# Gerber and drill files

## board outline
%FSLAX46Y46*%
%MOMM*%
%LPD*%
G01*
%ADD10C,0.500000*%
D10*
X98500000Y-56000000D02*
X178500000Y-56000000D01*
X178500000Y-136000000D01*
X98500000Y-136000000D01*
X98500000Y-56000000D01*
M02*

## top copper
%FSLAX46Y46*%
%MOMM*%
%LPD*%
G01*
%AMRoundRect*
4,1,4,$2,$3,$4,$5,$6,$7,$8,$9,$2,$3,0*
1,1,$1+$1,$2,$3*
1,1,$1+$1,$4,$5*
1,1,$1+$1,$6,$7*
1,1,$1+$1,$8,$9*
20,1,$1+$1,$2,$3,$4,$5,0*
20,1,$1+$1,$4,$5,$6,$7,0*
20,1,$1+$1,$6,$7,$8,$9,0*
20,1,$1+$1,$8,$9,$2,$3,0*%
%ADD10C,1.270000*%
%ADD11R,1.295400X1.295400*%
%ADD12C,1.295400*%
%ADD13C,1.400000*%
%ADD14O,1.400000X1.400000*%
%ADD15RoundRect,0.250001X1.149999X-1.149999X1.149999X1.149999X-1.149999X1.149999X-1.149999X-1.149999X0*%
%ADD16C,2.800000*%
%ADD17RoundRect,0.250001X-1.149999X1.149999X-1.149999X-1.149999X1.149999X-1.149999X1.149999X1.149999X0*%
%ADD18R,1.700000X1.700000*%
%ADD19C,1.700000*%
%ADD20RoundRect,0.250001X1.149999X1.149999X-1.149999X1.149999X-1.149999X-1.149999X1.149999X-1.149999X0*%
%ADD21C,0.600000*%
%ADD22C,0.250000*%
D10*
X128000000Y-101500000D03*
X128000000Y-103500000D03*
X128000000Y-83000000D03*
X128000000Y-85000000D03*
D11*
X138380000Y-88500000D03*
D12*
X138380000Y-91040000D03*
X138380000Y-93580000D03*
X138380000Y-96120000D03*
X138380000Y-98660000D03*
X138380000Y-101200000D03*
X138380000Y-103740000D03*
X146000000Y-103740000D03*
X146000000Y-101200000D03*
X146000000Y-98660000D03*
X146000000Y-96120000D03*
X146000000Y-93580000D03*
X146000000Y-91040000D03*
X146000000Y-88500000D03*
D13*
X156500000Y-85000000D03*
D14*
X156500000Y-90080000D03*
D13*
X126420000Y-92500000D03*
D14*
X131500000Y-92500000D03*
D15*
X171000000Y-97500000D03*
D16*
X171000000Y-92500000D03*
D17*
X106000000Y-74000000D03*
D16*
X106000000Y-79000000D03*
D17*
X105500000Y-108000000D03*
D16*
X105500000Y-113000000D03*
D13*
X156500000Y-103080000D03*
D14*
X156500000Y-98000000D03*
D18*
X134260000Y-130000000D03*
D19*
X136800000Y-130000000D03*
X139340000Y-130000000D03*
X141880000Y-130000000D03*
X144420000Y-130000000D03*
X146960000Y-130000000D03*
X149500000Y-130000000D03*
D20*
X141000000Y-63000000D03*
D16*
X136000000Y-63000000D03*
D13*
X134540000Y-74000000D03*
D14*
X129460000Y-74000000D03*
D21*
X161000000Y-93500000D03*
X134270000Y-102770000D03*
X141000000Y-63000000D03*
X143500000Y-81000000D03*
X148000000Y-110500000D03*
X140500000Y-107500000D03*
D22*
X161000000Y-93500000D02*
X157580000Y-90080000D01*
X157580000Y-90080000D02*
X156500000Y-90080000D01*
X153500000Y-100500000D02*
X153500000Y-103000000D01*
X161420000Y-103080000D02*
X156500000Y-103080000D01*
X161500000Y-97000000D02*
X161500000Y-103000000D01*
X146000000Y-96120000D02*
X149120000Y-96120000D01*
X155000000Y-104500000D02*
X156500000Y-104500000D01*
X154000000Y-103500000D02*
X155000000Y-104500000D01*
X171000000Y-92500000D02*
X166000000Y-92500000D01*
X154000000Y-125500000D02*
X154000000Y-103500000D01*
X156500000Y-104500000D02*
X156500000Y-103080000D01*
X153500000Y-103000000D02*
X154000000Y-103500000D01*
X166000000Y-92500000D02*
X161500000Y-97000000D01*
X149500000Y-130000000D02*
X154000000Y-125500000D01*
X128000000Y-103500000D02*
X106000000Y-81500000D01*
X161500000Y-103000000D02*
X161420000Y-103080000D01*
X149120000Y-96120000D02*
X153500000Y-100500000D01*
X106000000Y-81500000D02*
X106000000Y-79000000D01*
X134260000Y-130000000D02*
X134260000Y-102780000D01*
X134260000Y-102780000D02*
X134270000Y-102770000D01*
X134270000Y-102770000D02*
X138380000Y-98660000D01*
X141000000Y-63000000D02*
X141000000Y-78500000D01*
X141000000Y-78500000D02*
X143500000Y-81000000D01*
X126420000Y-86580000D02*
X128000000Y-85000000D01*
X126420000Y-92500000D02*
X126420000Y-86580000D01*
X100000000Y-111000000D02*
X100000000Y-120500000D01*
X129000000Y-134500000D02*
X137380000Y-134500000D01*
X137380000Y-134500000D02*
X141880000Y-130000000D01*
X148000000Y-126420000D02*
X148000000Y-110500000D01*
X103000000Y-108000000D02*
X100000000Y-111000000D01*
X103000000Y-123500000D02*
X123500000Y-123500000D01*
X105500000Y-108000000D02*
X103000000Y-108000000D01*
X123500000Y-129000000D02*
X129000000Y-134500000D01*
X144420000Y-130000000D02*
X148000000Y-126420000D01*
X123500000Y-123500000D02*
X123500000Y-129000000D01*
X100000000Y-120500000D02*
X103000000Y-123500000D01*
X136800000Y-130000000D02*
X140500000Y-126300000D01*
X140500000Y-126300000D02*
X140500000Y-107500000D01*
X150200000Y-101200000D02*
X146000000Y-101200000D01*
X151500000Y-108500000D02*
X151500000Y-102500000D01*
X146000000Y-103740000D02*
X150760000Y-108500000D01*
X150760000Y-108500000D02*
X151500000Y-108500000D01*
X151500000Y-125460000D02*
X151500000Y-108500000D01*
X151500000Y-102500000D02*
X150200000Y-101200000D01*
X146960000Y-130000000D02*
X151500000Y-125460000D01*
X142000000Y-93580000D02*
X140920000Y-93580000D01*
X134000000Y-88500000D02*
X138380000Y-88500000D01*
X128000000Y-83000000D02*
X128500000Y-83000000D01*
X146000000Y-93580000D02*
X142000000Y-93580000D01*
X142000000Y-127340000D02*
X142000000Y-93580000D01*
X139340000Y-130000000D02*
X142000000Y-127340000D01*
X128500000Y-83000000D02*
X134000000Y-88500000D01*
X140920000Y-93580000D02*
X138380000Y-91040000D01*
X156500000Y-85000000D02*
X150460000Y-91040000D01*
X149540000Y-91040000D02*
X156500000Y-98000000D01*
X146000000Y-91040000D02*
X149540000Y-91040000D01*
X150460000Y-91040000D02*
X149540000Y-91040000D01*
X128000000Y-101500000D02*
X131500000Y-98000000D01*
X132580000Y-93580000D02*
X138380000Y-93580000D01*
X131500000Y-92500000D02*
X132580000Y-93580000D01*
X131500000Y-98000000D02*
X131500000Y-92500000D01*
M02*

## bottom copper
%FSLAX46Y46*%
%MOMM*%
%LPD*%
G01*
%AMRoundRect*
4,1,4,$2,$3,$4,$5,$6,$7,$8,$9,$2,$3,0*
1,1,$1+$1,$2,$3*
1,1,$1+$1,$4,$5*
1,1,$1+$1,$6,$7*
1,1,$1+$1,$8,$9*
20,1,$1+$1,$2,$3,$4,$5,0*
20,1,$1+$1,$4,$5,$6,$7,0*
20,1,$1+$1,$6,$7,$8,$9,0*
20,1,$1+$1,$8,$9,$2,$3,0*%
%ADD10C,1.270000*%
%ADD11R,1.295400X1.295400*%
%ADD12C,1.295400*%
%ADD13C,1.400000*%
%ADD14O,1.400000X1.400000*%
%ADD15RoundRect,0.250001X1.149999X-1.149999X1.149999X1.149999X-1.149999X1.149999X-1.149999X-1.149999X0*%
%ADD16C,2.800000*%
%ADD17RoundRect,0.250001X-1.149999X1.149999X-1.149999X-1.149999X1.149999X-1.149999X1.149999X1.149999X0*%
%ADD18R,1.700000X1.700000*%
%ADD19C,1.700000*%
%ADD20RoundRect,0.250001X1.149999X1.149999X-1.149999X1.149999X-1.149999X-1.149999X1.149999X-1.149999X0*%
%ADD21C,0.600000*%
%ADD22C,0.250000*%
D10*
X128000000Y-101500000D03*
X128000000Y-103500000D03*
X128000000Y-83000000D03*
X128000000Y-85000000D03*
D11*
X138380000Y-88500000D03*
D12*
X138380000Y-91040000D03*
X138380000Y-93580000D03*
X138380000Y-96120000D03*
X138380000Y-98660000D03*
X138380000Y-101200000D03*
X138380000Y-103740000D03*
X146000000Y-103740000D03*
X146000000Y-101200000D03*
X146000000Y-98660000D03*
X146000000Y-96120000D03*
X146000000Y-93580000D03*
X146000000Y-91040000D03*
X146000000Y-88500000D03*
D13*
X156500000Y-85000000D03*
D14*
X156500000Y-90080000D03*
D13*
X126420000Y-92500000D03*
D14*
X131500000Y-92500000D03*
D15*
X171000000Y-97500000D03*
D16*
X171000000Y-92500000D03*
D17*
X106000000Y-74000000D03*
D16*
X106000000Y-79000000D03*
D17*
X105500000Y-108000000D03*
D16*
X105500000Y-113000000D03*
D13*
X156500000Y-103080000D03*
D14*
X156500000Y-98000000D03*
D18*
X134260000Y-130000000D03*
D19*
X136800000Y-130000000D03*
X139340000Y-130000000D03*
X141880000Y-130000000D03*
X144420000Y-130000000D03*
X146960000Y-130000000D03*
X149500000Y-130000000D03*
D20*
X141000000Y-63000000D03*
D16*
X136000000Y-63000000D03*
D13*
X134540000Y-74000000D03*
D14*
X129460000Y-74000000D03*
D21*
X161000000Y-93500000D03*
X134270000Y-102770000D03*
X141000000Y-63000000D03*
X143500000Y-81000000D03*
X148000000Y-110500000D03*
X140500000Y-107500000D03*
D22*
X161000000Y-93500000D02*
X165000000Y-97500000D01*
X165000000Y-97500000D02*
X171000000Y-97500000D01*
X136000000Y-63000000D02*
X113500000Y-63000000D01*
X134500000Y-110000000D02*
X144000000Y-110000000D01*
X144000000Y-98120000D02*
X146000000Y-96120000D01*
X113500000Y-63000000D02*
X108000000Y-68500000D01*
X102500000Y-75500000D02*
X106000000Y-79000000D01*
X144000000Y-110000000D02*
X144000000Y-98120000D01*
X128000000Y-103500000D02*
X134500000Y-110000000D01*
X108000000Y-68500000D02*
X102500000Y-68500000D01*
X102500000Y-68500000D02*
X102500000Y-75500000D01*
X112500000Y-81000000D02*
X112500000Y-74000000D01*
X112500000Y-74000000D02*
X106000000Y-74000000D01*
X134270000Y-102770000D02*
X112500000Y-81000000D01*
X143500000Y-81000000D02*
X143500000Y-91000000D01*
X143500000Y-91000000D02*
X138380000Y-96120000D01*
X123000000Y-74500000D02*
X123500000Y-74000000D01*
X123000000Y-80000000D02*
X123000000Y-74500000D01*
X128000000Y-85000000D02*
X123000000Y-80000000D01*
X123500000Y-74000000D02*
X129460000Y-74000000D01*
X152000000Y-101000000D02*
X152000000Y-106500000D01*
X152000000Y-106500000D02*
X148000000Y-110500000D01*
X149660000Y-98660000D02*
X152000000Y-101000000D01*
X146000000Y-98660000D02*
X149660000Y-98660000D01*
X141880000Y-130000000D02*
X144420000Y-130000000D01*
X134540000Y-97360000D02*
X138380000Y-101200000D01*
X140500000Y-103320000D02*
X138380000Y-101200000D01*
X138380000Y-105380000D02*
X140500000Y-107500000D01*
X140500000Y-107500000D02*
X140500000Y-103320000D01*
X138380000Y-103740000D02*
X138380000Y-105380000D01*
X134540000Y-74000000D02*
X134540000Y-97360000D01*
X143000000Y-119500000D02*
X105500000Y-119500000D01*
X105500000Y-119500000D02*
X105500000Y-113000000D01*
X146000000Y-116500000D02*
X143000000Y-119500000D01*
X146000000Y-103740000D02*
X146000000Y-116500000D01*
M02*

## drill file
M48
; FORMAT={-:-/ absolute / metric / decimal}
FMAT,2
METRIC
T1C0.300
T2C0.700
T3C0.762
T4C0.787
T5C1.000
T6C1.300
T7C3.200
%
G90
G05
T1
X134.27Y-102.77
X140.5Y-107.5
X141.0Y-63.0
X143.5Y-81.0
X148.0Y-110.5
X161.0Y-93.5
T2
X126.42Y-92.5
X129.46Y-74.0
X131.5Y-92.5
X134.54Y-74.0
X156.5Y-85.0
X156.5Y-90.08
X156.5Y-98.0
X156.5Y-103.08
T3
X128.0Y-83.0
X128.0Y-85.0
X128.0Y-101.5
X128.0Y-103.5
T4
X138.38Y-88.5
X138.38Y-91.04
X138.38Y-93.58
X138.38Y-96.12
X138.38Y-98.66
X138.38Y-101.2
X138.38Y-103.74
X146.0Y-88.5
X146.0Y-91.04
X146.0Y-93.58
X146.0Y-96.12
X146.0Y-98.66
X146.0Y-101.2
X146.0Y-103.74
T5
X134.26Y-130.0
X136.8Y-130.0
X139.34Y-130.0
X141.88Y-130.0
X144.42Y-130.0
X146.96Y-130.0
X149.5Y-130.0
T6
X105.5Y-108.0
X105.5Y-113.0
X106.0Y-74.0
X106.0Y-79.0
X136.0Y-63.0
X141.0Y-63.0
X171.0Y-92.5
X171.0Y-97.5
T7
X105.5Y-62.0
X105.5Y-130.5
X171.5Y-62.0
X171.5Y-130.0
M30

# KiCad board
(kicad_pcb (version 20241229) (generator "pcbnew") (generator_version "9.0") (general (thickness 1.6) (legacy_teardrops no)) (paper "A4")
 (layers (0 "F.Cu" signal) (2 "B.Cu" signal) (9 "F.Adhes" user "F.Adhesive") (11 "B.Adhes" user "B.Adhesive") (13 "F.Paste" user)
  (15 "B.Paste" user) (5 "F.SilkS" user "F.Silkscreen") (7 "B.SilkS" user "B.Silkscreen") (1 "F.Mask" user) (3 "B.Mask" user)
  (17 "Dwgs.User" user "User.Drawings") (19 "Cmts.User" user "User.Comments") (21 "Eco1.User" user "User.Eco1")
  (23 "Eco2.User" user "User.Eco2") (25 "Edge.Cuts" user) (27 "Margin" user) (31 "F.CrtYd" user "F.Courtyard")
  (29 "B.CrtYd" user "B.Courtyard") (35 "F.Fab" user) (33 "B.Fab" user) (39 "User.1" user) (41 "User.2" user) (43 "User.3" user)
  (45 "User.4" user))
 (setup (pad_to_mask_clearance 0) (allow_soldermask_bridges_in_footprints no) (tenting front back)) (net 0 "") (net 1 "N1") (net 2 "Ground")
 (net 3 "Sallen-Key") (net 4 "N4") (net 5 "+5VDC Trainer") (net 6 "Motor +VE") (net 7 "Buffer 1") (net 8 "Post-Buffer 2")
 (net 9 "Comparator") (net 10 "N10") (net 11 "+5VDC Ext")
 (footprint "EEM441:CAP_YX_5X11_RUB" (layer "F.Cu") (at 128 101.5 -90)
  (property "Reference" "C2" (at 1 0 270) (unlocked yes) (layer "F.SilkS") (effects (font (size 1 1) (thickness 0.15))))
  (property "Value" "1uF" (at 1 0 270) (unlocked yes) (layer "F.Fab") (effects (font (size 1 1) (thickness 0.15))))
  (pad "1" thru_hole circle (at 0 0 270) (size 1.27 1.27) (drill 0.762) (layers "*.Cu" "*.Mask") (remove_unused_layers no) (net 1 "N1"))
  (pad "2" thru_hole circle (at 2 0 270) (size 1.27 1.27) (drill 0.762) (layers "*.Cu" "*.Mask") (remove_unused_layers no) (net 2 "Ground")))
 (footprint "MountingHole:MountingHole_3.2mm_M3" (layer "F.Cu") (at 105.5 62)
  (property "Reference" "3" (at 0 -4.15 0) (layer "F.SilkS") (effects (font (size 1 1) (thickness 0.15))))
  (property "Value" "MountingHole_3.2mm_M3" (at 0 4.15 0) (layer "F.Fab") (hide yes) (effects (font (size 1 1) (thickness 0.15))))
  (pad "" np_thru_hole circle (at 0 0) (size 3.2 3.2) (drill 3.2) (layers "*.Cu" "*.Mask")))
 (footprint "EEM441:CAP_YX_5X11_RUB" (layer "F.Cu") (at 128 83 -90)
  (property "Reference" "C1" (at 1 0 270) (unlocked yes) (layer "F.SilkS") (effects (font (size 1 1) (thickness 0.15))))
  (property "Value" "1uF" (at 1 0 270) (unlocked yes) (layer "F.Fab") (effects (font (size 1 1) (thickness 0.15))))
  (pad "1" thru_hole circle (at 0 0 270) (size 1.27 1.27) (drill 0.762) (layers "*.Cu" "*.Mask") (remove_unused_layers no)
   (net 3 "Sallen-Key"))
  (pad "2" thru_hole circle (at 2 0 270) (size 1.27 1.27) (drill 0.762) (layers "*.Cu" "*.Mask") (remove_unused_layers no) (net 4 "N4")))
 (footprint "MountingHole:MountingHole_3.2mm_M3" (layer "F.Cu") (at 105.5 130.5)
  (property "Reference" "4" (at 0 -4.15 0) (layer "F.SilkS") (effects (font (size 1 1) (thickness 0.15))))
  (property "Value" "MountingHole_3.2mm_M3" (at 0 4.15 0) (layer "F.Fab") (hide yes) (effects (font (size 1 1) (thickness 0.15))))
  (pad "" np_thru_hole circle (at 0 0) (size 3.2 3.2) (drill 3.2) (layers "*.Cu" "*.Mask")))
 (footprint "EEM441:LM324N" (layer "F.Cu") (at 138.38 88.5)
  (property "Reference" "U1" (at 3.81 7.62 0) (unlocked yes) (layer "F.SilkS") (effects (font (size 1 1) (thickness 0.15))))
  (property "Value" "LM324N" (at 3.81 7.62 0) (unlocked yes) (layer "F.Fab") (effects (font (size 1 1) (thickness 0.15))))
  (pad "1" thru_hole rect (at 0 0) (size 1.2954 1.2954) (drill 0.7874) (layers "*.Cu" "*.Mask") (remove_unused_layers no)
   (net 3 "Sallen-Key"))
  (pad "2" thru_hole circle (at 0 2.54) (size 1.2954 1.2954) (drill 0.7874) (layers "*.Cu" "*.Mask") (remove_unused_layers no)
   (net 3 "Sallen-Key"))
  (pad "3" thru_hole circle (at 0 5.08) (size 1.2954 1.2954) (drill 0.7874) (layers "*.Cu" "*.Mask") (remove_unused_layers no) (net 1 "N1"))
  (pad "4" thru_hole circle (at 0 7.62) (size 1.2954 1.2954) (drill 0.7874) (layers "*.Cu" "*.Mask") (remove_unused_layers no)
   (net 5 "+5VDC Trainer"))
  (pad "5" thru_hole circle (at 0 10.16) (size 1.2954 1.2954) (drill 0.7874) (layers "*.Cu" "*.Mask") (remove_unused_layers no)
   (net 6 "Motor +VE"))
  (pad "6" thru_hole circle (at 0 12.7) (size 1.2954 1.2954) (drill 0.7874) (layers "*.Cu" "*.Mask") (remove_unused_layers no)
   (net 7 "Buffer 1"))
  (pad "7" thru_hole circle (at 0 15.24) (size 1.2954 1.2954) (drill 0.7874) (layers "*.Cu" "*.Mask") (remove_unused_layers no)
   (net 7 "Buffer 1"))
  (pad "8" thru_hole circle (at 7.62 15.24) (size 1.2954 1.2954) (drill 0.7874) (layers "*.Cu" "*.Mask") (remove_unused_layers no)
   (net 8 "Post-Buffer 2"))
  (pad "9" thru_hole circle (at 7.62 12.7) (size 1.2954 1.2954) (drill 0.7874) (layers "*.Cu" "*.Mask") (remove_unused_layers no)
   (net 8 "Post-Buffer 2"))
  (pad "10" thru_hole circle (at 7.62 10.16) (size 1.2954 1.2954) (drill 0.7874) (layers "*.Cu" "*.Mask") (remove_unused_layers no)
   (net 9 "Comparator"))
  (pad "11" thru_hole circle (at 7.62 7.62) (size 1.2954 1.2954) (drill 0.7874) (layers "*.Cu" "*.Mask") (remove_unused_layers no)
   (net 2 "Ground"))
  (pad "12" thru_hole circle (at 7.62 5.08) (size 1.2954 1.2954) (drill 0.7874) (layers "*.Cu" "*.Mask") (remove_unused_layers no)
   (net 3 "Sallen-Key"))
  (pad "13" thru_hole circle (at 7.62 2.54) (size 1.2954 1.2954) (drill 0.7874) (layers "*.Cu" "*.Mask") (remove_unused_layers no)
   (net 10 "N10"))
  (pad "14" thru_hole circle (at 7.62 0) (size 1.2954 1.2954) (drill 0.7874) (layers "*.Cu" "*.Mask") (remove_unused_layers no)
   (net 9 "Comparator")))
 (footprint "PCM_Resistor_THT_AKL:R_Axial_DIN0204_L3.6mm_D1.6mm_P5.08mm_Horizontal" (layer "F.Cu") (at 156.5 85 -90)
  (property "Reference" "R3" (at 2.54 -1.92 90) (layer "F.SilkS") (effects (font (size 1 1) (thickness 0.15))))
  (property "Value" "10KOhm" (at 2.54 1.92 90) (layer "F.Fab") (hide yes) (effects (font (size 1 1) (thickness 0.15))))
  (pad "1" thru_hole circle (at 0 0 270) (size 1.4 1.4) (drill 0.7) (layers "*.Cu" "*.Mask") (remove_unused_layers no) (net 10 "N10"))
  (pad "2" thru_hole oval (at 5.08 0 270) (size 1.4 1.4) (drill 0.7) (layers "*.Cu" "*.Mask") (remove_unused_layers no) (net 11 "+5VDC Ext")))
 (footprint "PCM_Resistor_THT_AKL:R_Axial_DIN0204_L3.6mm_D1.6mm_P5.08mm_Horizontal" (layer "F.Cu") (at 126.42 92.5)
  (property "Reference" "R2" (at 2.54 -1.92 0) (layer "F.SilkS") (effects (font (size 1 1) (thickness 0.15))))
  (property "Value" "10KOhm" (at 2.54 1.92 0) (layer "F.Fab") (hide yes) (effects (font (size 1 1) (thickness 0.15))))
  (pad "1" thru_hole circle (at 0 0) (size 1.4 1.4) (drill 0.7) (layers "*.Cu" "*.Mask") (remove_unused_layers no) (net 4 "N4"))
  (pad "2" thru_hole oval (at 5.08 0) (size 1.4 1.4) (drill 0.7) (layers "*.Cu" "*.Mask") (remove_unused_layers no) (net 1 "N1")))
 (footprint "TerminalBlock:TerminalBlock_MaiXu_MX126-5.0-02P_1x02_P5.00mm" (layer "F.Cu") (at 171 97.5 90)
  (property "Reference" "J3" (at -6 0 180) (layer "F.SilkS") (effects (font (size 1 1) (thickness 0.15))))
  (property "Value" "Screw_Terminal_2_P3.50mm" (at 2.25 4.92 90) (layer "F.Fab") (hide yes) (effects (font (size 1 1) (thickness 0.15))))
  (pad "1" thru_hole roundrect (at 0 0 90) (size 2.8 2.8) (drill 1.3) (layers "*.Cu" "*.Mask") (remove_unused_layers no)
   (roundrect_rratio 0.089286) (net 11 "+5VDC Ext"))
  (pad "2" thru_hole circle (at 5 0 90) (size 2.8 2.8) (drill 1.3) (layers "*.Cu" "*.Mask") (remove_unused_layers no) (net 2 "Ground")))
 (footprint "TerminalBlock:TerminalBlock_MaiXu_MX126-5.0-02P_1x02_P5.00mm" (layer "F.Cu") (at 106 74 -90)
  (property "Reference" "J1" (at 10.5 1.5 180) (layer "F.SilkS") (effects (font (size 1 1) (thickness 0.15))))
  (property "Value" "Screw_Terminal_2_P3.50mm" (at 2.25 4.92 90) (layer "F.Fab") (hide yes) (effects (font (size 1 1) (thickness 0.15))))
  (pad "1" thru_hole roundrect (at 0 0 270) (size 2.8 2.8) (drill 1.3) (layers "*.Cu" "*.Mask") (remove_unused_layers no)
   (roundrect_rratio 0.089286) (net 6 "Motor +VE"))
  (pad "2" thru_hole circle (at 5 0 270) (size 2.8 2.8) (drill 1.3) (layers "*.Cu" "*.Mask") (remove_unused_layers no) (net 2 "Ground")))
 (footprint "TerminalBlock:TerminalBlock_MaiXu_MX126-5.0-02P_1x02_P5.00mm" (layer "F.Cu") (at 105.5 108 -90)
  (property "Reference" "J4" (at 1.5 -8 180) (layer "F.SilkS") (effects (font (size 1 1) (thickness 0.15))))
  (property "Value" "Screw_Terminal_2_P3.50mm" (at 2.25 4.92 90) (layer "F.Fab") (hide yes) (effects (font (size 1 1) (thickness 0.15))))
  (pad "1" thru_hole roundrect (at 0 0 270) (size 2.8 2.8) (drill 1.3) (layers "*.Cu" "*.Mask") (remove_unused_layers no)
   (roundrect_rratio 0.089286) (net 9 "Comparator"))
  (pad "2" thru_hole circle (at 5 0 270) (size 2.8 2.8) (drill 1.3) (layers "*.Cu" "*.Mask") (remove_unused_layers no)
   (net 8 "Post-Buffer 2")))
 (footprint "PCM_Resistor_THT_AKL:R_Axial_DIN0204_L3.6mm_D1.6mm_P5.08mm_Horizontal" (layer "F.Cu") (at 156.5 103.08 90)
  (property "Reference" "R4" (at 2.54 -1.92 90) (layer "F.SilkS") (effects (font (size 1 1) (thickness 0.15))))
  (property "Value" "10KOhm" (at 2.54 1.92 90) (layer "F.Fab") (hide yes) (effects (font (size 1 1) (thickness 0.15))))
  (pad "1" thru_hole circle (at 0 0 90) (size 1.4 1.4) (drill 0.7) (layers "*.Cu" "*.Mask") (remove_unused_layers no) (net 2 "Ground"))
  (pad "2" thru_hole oval (at 5.08 0 90) (size 1.4 1.4) (drill 0.7) (layers "*.Cu" "*.Mask") (remove_unused_layers no) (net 10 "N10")))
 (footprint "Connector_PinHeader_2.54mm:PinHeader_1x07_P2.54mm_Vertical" (layer "F.Cu") (at 134.26 130 90)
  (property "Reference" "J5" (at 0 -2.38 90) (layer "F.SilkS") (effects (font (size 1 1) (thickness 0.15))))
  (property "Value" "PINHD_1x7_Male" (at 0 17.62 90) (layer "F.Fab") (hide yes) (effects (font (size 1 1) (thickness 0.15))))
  (pad "1" thru_hole rect (at 0 0 90) (size 1.7 1.7) (drill 1) (layers "*.Cu" "*.Mask") (remove_unused_layers no) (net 6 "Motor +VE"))
  (pad "2" thru_hole circle (at 0 2.54 90) (size 1.7 1.7) (drill 1) (layers "*.Cu" "*.Mask") (remove_unused_layers no) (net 7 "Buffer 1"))
  (pad "3" thru_hole circle (at 0 5.08 90) (size 1.7 1.7) (drill 1) (layers "*.Cu" "*.Mask") (remove_unused_layers no) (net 3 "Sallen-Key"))
  (pad "4" thru_hole circle (at 0 7.62 90) (size 1.7 1.7) (drill 1) (layers "*.Cu" "*.Mask") (remove_unused_layers no) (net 9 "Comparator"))
  (pad "5" thru_hole circle (at 0 10.16 90) (size 1.7 1.7) (drill 1) (layers "*.Cu" "*.Mask") (remove_unused_layers no) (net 9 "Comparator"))
  (pad "6" thru_hole circle (at 0 12.7 90) (size 1.7 1.7) (drill 1) (layers "*.Cu" "*.Mask") (remove_unused_layers no)
   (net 8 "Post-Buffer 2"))
  (pad "7" thru_hole circle (at 0 15.24 90) (size 1.7 1.7) (drill 1) (layers "*.Cu" "*.Mask") (remove_unused_layers no) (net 2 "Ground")))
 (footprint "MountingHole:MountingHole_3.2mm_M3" (layer "F.Cu") (at 171.5 130)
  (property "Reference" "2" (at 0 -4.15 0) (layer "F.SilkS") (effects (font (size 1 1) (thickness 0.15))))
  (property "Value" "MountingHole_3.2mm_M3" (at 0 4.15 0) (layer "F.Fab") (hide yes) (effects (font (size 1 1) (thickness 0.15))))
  (pad "" np_thru_hole circle (at 0 0) (size 3.2 3.2) (drill 3.2) (layers "*.Cu" "*.Mask")))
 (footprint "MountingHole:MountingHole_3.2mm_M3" (layer "F.Cu") (at 171.5 62)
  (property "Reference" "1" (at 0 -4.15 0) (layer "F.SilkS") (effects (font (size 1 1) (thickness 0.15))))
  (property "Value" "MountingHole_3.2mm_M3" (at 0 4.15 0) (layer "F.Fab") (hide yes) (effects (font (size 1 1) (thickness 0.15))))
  (pad "" np_thru_hole circle (at 0 0) (size 3.2 3.2) (drill 3.2) (layers "*.Cu" "*.Mask")))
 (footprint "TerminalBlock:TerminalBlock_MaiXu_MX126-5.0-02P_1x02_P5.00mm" (layer "F.Cu") (at 141 63 180)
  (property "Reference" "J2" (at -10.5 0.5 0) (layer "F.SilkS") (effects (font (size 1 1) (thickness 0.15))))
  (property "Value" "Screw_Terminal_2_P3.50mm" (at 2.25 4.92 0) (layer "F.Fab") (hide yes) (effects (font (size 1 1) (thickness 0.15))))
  (pad "1" thru_hole roundrect (at 0 0 180) (size 2.8 2.8) (drill 1.3) (layers "*.Cu" "*.Mask") (remove_unused_layers no)
   (roundrect_rratio 0.089286) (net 5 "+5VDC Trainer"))
  (pad "2" thru_hole circle (at 5 0 180) (size 2.8 2.8) (drill 1.3) (layers "*.Cu" "*.Mask") (remove_unused_layers no) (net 2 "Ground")))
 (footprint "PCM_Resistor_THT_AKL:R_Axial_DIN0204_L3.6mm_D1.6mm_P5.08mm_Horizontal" (layer "F.Cu") (at 134.54 74 180)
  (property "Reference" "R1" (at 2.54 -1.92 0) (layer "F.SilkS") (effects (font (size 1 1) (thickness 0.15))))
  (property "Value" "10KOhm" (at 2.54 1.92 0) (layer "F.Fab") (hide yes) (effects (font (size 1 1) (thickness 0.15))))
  (pad "1" thru_hole circle (at 0 0 180) (size 1.4 1.4) (drill 0.7) (layers "*.Cu" "*.Mask") (remove_unused_layers no) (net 7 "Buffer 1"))
  (pad "2" thru_hole oval (at 5.08 0 180) (size 1.4 1.4) (drill 0.7) (layers "*.Cu" "*.Mask") (remove_unused_layers no) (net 4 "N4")))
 (gr_rect (start 98.5 56) (end 178.5 136) (stroke (width 0.5) (type solid)) (fill no) (layer "Edge.Cuts"))
 (segment (start 161 93.5) (end 157.58 90.08) (width 0.25) (layer "F.Cu") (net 11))
 (segment (start 157.58 90.08) (end 156.5 90.08) (width 0.25) (layer "F.Cu") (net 11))
 (via (at 161 93.5) (size 0.6) (drill 0.3) (layers "F.Cu" "B.Cu") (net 11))
 (segment (start 161 93.5) (end 165 97.5) (width 0.25) (layer "B.Cu") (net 11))
 (segment (start 165 97.5) (end 171 97.5) (width 0.25) (layer "B.Cu") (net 11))
 (segment (start 153.5 100.5) (end 153.5 103) (width 0.25) (layer "F.Cu") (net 2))
 (segment (start 161.42 103.08) (end 156.5 103.08) (width 0.25) (layer "F.Cu") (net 2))
 (segment (start 161.5 97) (end 161.5 103) (width 0.25) (layer "F.Cu") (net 2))
 (segment (start 146 96.12) (end 149.12 96.12) (width 0.25) (layer "F.Cu") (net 2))
 (segment (start 155 104.5) (end 156.5 104.5) (width 0.25) (layer "F.Cu") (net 2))
 (segment (start 154 103.5) (end 155 104.5) (width 0.25) (layer "F.Cu") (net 2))
 (segment (start 171 92.5) (end 166 92.5) (width 0.25) (layer "F.Cu") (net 2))
 (segment (start 154 125.5) (end 154 103.5) (width 0.25) (layer "F.Cu") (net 2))
 (segment (start 156.5 104.5) (end 156.5 103.08) (width 0.25) (layer "F.Cu") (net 2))
 (segment (start 153.5 103) (end 154 103.5) (width 0.25) (layer "F.Cu") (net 2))
 (segment (start 166 92.5) (end 161.5 97) (width 0.25) (layer "F.Cu") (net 2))
 (segment (start 149.5 130) (end 154 125.5) (width 0.25) (layer "F.Cu") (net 2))
 (segment (start 128 103.5) (end 106 81.5) (width 0.25) (layer "F.Cu") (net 2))
 (segment (start 161.5 103) (end 161.42 103.08) (width 0.25) (layer "F.Cu") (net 2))
 (segment (start 149.12 96.12) (end 153.5 100.5) (width 0.25) (layer "F.Cu") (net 2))
 (segment (start 106 81.5) (end 106 79) (width 0.25) (layer "F.Cu") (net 2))
 (segment (start 136 63) (end 113.5 63) (width 0.25) (layer "B.Cu") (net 2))
 (segment (start 134.5 110) (end 144 110) (width 0.25) (layer "B.Cu") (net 2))
 (segment (start 144 98.12) (end 146 96.12) (width 0.25) (layer "B.Cu") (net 2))
 (segment (start 113.5 63) (end 108 68.5) (width 0.25) (layer "B.Cu") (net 2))
 (segment (start 102.5 75.5) (end 106 79) (width 0.25) (layer "B.Cu") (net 2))
 (segment (start 144 110) (end 144 98.12) (width 0.25) (layer "B.Cu") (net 2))
 (segment (start 128 103.5) (end 134.5 110) (width 0.25) (layer "B.Cu") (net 2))
 (segment (start 108 68.5) (end 102.5 68.5) (width 0.25) (layer "B.Cu") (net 2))
 (segment (start 102.5 68.5) (end 102.5 75.5) (width 0.25) (layer "B.Cu") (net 2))
 (segment (start 134.26 130) (end 134.26 102.78) (width 0.25) (layer "F.Cu") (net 6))
 (segment (start 134.26 102.78) (end 134.27 102.77) (width 0.25) (layer "F.Cu") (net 6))
 (segment (start 134.27 102.77) (end 138.38 98.66) (width 0.25) (layer "F.Cu") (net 6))
 (via (at 134.27 102.77) (size 0.6) (drill 0.3) (layers "F.Cu" "B.Cu") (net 6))
 (segment (start 112.5 81) (end 112.5 74) (width 0.25) (layer "B.Cu") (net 6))
 (segment (start 112.5 74) (end 106 74) (width 0.25) (layer "B.Cu") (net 6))
 (segment (start 134.27 102.77) (end 112.5 81) (width 0.25) (layer "B.Cu") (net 6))
 (segment (start 141 63) (end 141 78.5) (width 0.25) (layer "F.Cu") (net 5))
 (segment (start 141 78.5) (end 143.5 81) (width 0.25) (layer "F.Cu") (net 5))
 (via (at 141 63) (size 0.6) (drill 0.3) (layers "F.Cu" "B.Cu") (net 5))
 (via (at 143.5 81) (size 0.6) (drill 0.3) (layers "F.Cu" "B.Cu") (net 5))
 (segment (start 143.5 81) (end 143.5 91) (width 0.25) (layer "B.Cu") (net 5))
 (segment (start 143.5 91) (end 138.38 96.12) (width 0.25) (layer "B.Cu") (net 5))
 (segment (start 126.42 86.58) (end 128 85) (width 0.25) (layer "F.Cu") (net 4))
 (segment (start 126.42 92.5) (end 126.42 86.58) (width 0.25) (layer "F.Cu") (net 4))
 (segment (start 123 74.5) (end 123.5 74) (width 0.25) (layer "B.Cu") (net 4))
 (segment (start 123 80) (end 123 74.5) (width 0.25) (layer "B.Cu") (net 4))
 (segment (start 128 85) (end 123 80) (width 0.25) (layer "B.Cu") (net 4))
 (segment (start 123.5 74) (end 129.46 74) (width 0.25) (layer "B.Cu") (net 4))
 (segment (start 100 111) (end 100 120.5) (width 0.25) (layer "F.Cu") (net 9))
 (segment (start 129 134.5) (end 137.38 134.5) (width 0.25) (layer "F.Cu") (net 9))
 (segment (start 137.38 134.5) (end 141.88 130) (width 0.25) (layer "F.Cu") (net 9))
 (segment (start 148 126.42) (end 148 110.5) (width 0.25) (layer "F.Cu") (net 9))
 (segment (start 103 108) (end 100 111) (width 0.25) (layer "F.Cu") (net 9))
 (segment (start 103 123.5) (end 123.5 123.5) (width 0.25) (layer "F.Cu") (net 9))
 (segment (start 105.5 108) (end 103 108) (width 0.25) (layer "F.Cu") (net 9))
 (segment (start 123.5 129) (end 129 134.5) (width 0.25) (layer "F.Cu") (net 9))
 (segment (start 144.42 130) (end 148 126.42) (width 0.25) (layer "F.Cu") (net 9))
 (segment (start 123.5 123.5) (end 123.5 129) (width 0.25) (layer "F.Cu") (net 9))
 (segment (start 100 120.5) (end 103 123.5) (width 0.25) (layer "F.Cu") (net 9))
 (via (at 148 110.5) (size 0.6) (drill 0.3) (layers "F.Cu" "B.Cu") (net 9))
 (segment (start 152 101) (end 152 106.5) (width 0.25) (layer "B.Cu") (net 9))
 (segment (start 152 106.5) (end 148 110.5) (width 0.25) (layer "B.Cu") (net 9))
 (segment (start 149.66 98.66) (end 152 101) (width 0.25) (layer "B.Cu") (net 9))
 (segment (start 146 98.66) (end 149.66 98.66) (width 0.25) (layer "B.Cu") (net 9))
 (segment (start 141.88 130) (end 144.42 130) (width 0.25) (layer "B.Cu") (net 9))
 (segment (start 136.8 130) (end 140.5 126.3) (width 0.25) (layer "F.Cu") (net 7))
 (segment (start 140.5 126.3) (end 140.5 107.5) (width 0.25) (layer "F.Cu") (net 7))
 (via (at 140.5 107.5) (size 0.6) (drill 0.3) (layers "F.Cu" "B.Cu") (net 7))
 (segment (start 134.54 97.36) (end 138.38 101.2) (width 0.25) (layer "B.Cu") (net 7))
 (segment (start 140.5 103.32) (end 138.38 101.2) (width 0.25) (layer "B.Cu") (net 7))
 (segment (start 138.38 105.38) (end 140.5 107.5) (width 0.25) (layer "B.Cu") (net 7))
 (segment (start 140.5 107.5) (end 140.5 103.32) (width 0.25) (layer "B.Cu") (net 7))
 (segment (start 138.38 103.74) (end 138.38 105.38) (width 0.25) (layer "B.Cu") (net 7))
 (segment (start 134.54 74) (end 134.54 97.36) (width 0.25) (layer "B.Cu") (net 7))
 (segment (start 150.2 101.2) (end 146 101.2) (width 0.25) (layer "F.Cu") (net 8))
 (segment (start 151.5 108.5) (end 151.5 102.5) (width 0.25) (layer "F.Cu") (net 8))
 (segment (start 146 103.74) (end 150.76 108.5) (width 0.25) (layer "F.Cu") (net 8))
 (segment (start 150.76 108.5) (end 151.5 108.5) (width 0.25) (layer "F.Cu") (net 8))
 (segment (start 151.5 125.46) (end 151.5 108.5) (width 0.25) (layer "F.Cu") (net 8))
 (segment (start 151.5 102.5) (end 150.2 101.2) (width 0.25) (layer "F.Cu") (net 8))
 (segment (start 146.96 130) (end 151.5 125.46) (width 0.25) (layer "F.Cu") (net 8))
 (segment (start 143 119.5) (end 105.5 119.5) (width 0.25) (layer "B.Cu") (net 8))
 (segment (start 105.5 119.5) (end 105.5 113) (width 0.25) (layer "B.Cu") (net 8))
 (segment (start 146 116.5) (end 143 119.5) (width 0.25) (layer "B.Cu") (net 8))
 (segment (start 146 103.74) (end 146 116.5) (width 0.25) (layer "B.Cu") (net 8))
 (segment (start 142 93.58) (end 140.92 93.58) (width 0.25) (layer "F.Cu") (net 3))
 (segment (start 134 88.5) (end 138.38 88.5) (width 0.25) (layer "F.Cu") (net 3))
 (segment (start 128 83) (end 128.5 83) (width 0.25) (layer "F.Cu") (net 3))
 (segment (start 146 93.58) (end 142 93.58) (width 0.25) (layer "F.Cu") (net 3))
 (segment (start 142 127.34) (end 142 93.58) (width 0.25) (layer "F.Cu") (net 3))
 (segment (start 139.34 130) (end 142 127.34) (width 0.25) (layer "F.Cu") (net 3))
 (segment (start 128.5 83) (end 134 88.5) (width 0.25) (layer "F.Cu") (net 3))
 (segment (start 140.92 93.58) (end 138.38 91.04) (width 0.25) (layer "F.Cu") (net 3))
 (segment (start 156.5 85) (end 150.46 91.04) (width 0.25) (layer "F.Cu") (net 10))
 (segment (start 149.54 91.04) (end 156.5 98) (width 0.25) (layer "F.Cu") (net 10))
 (segment (start 146 91.04) (end 149.54 91.04) (width 0.25) (layer "F.Cu") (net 10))
 (segment (start 150.46 91.04) (end 149.54 91.04) (width 0.25) (layer "F.Cu") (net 10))
 (segment (start 128 101.5) (end 131.5 98) (width 0.25) (layer "F.Cu") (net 1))
 (segment (start 132.58 93.58) (end 138.38 93.58) (width 0.25) (layer "F.Cu") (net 1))
 (segment (start 131.5 92.5) (end 132.58 93.58) (width 0.25) (layer "F.Cu") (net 1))
 (segment (start 131.5 98) (end 131.5 92.5) (width 0.25) (layer "F.Cu") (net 1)))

